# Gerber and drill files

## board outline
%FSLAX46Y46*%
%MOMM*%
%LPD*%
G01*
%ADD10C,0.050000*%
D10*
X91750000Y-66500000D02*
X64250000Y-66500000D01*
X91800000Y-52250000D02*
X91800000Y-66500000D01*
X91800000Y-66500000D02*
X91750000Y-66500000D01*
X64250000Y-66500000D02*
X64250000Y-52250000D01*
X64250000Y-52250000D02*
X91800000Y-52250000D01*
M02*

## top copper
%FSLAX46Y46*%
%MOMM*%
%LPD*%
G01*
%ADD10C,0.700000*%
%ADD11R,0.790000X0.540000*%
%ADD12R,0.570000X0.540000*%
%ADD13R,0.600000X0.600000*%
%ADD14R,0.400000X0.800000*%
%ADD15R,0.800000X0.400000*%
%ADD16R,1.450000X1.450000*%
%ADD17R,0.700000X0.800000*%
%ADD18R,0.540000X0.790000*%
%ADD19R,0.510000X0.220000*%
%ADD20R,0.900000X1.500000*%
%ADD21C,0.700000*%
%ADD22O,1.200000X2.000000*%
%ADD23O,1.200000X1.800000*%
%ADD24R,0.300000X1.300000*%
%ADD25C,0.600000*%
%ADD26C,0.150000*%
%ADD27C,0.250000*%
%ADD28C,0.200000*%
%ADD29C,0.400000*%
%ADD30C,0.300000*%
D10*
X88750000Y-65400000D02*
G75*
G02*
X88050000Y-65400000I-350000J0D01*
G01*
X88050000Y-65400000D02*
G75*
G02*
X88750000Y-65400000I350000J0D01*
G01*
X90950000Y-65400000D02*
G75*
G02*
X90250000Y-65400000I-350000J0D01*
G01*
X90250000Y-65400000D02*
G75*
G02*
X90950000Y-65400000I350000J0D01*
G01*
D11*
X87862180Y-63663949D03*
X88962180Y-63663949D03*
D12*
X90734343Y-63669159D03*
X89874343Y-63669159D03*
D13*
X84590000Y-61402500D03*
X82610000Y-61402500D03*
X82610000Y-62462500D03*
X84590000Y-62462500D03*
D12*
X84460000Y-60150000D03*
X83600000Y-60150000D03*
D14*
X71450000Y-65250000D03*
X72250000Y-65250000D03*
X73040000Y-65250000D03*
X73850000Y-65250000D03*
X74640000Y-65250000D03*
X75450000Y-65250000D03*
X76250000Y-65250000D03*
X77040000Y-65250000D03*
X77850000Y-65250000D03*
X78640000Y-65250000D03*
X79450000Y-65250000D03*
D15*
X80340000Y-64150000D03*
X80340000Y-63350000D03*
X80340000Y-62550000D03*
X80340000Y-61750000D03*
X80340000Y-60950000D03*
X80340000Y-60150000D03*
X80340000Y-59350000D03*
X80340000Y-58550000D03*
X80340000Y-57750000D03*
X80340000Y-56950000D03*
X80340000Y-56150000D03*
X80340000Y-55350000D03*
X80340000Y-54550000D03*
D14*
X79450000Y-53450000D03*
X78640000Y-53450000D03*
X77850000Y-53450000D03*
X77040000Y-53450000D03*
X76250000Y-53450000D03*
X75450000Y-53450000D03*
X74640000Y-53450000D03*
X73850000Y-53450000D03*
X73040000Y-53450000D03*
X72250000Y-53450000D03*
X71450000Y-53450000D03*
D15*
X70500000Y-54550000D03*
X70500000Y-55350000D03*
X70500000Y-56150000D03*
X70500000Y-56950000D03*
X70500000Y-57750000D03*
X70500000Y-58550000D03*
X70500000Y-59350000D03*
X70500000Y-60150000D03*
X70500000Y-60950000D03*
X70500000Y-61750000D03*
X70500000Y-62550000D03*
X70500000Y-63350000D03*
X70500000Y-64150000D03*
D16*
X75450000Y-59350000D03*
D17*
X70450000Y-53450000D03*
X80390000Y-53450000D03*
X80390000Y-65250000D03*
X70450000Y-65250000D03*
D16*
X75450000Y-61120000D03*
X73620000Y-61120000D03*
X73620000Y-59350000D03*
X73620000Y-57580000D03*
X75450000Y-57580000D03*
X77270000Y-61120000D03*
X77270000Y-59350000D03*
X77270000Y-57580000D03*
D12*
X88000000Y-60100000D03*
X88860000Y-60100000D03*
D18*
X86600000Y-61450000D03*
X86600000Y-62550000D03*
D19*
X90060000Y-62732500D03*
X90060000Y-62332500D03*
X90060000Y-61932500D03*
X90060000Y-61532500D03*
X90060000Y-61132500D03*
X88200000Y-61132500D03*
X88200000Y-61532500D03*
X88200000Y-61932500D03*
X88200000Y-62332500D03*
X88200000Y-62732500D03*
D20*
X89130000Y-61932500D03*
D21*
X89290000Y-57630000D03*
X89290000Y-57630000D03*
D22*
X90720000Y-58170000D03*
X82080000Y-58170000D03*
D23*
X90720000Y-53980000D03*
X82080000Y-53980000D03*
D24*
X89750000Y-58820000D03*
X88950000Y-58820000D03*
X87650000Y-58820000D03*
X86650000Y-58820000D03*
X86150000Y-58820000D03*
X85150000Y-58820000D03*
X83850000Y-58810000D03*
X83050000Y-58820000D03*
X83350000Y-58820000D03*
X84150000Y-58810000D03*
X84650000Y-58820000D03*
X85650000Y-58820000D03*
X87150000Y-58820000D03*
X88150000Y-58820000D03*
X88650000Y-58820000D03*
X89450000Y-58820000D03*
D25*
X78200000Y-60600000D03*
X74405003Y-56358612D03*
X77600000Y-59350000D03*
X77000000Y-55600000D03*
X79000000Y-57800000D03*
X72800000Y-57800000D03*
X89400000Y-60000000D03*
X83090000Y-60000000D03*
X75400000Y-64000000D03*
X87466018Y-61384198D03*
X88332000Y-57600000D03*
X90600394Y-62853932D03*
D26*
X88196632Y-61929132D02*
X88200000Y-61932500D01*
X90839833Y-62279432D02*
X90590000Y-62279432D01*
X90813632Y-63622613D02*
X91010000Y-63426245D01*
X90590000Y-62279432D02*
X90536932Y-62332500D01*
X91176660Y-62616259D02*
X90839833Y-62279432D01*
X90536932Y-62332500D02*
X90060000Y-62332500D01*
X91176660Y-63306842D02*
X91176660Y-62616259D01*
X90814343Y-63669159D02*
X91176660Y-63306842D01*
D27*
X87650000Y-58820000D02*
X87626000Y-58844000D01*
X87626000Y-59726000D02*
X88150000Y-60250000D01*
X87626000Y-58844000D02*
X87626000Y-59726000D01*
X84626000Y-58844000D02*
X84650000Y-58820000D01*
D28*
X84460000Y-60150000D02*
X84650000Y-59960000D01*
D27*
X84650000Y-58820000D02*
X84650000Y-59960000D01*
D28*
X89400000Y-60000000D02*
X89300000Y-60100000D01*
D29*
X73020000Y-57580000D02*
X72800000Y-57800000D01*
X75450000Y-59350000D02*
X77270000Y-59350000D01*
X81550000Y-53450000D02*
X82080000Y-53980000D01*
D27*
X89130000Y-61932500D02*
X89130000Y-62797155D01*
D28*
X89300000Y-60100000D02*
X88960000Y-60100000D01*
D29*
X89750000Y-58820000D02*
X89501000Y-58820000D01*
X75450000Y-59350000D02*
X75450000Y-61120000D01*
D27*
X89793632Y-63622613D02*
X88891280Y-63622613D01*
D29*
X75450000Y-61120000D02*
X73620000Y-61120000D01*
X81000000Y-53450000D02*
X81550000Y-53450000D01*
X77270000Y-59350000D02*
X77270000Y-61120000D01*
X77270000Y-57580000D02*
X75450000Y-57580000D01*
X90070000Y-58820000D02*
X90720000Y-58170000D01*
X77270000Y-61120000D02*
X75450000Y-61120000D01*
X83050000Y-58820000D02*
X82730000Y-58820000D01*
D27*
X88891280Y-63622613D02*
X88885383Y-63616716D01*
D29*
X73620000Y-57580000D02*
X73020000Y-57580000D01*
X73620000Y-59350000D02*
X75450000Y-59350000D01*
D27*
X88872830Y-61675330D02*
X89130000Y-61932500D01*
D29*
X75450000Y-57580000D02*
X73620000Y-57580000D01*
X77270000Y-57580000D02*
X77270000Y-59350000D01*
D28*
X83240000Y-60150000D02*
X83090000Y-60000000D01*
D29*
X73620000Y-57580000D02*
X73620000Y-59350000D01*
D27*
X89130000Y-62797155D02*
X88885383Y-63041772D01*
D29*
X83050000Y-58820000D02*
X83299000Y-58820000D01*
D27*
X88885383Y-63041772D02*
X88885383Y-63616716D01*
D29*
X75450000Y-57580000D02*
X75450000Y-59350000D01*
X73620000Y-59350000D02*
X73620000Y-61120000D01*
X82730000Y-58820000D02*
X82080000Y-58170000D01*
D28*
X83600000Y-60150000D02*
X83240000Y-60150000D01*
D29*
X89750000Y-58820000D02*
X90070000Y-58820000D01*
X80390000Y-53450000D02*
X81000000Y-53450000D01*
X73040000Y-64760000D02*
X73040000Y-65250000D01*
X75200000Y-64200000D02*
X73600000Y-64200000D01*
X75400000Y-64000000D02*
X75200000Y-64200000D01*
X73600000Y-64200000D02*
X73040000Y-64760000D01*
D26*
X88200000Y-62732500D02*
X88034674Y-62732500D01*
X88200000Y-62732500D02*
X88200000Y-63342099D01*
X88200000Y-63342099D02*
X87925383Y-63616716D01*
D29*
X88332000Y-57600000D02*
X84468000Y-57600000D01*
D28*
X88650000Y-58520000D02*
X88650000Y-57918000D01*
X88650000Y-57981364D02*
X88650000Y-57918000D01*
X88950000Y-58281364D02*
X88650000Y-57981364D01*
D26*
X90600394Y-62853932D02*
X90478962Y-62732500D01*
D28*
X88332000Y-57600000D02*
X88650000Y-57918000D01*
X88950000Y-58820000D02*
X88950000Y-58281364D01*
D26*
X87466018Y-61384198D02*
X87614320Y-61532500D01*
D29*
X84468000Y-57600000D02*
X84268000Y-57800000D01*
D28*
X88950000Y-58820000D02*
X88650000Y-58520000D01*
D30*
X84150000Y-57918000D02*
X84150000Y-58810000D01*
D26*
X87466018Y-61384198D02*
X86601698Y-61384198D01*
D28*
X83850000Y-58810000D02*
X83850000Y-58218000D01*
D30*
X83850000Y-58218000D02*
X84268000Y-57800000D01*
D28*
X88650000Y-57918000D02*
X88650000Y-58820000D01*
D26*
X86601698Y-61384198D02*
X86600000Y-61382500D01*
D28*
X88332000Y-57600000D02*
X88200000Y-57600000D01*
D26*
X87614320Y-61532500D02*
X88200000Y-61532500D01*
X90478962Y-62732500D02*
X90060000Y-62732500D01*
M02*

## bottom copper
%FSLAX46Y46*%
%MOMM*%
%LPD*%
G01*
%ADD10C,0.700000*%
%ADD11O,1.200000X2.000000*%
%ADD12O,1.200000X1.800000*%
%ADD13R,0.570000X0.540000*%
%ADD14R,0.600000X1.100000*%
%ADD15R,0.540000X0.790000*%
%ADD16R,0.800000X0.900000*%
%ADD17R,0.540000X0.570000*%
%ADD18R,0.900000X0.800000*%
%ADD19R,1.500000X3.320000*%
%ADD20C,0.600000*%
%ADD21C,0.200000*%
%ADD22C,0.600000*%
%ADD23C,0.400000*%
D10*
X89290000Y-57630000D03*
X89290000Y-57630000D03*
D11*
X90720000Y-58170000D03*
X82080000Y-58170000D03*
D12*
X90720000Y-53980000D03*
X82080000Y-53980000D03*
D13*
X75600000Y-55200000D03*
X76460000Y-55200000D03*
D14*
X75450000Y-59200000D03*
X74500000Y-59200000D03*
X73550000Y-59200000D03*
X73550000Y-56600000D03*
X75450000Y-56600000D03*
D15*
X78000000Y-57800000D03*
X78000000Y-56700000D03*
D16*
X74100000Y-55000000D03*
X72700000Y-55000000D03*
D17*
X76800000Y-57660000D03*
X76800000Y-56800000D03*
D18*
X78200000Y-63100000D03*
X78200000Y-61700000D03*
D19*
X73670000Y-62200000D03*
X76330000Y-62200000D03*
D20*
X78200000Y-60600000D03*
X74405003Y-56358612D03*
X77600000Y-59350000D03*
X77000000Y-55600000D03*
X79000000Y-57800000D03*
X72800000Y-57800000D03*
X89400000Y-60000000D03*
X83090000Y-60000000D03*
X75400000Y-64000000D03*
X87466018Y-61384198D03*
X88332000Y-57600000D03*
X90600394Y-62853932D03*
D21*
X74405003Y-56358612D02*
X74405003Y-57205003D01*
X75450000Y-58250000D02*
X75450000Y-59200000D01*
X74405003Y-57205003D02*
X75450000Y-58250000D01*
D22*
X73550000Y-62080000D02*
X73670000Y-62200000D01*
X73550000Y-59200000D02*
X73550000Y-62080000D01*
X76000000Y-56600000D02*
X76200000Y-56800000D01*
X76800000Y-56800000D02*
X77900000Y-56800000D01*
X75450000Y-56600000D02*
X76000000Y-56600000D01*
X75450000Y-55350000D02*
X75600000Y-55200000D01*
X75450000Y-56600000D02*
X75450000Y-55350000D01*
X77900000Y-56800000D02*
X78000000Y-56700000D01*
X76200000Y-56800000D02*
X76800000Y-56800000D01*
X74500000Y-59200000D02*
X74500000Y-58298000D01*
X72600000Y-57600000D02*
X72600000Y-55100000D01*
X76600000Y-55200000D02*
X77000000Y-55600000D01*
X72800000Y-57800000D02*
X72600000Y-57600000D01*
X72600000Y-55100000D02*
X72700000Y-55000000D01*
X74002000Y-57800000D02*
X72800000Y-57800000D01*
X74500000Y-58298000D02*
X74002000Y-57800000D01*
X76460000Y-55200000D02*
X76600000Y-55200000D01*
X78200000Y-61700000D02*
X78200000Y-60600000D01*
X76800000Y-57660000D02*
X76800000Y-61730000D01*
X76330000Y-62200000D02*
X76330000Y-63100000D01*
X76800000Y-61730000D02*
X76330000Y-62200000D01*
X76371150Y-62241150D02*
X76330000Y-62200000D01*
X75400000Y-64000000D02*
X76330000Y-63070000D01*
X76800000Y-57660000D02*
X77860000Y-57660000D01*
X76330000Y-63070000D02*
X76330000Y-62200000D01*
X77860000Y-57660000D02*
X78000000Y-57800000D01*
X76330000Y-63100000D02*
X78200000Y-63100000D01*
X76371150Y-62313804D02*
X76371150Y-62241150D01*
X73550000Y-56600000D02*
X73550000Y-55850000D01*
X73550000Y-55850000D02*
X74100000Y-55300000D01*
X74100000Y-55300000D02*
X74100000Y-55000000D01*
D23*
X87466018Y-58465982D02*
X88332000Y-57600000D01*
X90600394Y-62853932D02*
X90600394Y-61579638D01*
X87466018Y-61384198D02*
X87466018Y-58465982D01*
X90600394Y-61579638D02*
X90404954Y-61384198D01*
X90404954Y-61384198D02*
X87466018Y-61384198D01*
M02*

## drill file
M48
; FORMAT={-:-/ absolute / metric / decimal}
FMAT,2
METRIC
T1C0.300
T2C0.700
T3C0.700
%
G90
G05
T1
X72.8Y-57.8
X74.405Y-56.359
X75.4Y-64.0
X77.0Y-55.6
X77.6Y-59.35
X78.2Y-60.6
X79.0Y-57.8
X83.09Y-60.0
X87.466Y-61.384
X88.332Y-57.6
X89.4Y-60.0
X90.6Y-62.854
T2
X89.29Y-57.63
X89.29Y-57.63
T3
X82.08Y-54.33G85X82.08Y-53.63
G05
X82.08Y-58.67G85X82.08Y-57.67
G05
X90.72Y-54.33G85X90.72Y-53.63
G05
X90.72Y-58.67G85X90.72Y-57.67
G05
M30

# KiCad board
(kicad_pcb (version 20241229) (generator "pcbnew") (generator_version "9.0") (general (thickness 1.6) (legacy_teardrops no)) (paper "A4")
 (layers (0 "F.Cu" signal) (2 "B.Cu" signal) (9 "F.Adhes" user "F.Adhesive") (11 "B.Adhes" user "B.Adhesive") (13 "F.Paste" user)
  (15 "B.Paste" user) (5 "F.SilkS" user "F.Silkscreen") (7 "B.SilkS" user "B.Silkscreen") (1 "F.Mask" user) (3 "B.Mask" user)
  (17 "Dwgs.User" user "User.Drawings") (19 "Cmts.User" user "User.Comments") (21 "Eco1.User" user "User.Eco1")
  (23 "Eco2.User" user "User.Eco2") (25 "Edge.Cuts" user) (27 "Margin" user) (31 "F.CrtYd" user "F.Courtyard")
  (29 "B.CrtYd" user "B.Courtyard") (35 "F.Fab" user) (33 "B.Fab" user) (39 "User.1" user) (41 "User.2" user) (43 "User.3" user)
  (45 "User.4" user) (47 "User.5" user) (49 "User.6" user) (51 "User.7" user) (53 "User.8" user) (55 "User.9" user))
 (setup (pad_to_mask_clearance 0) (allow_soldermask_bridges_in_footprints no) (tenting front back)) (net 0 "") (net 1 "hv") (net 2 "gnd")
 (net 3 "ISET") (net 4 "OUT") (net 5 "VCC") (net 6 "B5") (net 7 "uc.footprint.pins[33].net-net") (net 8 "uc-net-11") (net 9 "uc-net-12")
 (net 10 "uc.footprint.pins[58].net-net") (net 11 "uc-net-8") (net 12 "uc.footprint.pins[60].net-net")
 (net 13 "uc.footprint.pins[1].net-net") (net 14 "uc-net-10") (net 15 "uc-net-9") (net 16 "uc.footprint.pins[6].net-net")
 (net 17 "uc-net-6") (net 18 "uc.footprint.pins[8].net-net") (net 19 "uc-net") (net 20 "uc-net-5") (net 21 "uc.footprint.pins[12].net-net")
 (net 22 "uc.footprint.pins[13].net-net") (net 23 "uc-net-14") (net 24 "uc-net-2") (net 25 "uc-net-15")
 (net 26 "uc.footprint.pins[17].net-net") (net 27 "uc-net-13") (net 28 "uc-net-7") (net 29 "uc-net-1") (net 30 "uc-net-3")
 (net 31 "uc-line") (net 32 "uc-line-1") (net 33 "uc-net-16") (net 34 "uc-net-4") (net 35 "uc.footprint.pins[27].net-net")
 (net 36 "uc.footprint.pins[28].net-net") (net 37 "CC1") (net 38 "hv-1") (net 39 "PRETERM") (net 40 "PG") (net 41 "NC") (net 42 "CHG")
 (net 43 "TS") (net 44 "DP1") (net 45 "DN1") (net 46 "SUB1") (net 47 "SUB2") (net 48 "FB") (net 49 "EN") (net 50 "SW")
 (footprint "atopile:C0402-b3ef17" (layer "F.Cu") (at 88.41218 63.663949)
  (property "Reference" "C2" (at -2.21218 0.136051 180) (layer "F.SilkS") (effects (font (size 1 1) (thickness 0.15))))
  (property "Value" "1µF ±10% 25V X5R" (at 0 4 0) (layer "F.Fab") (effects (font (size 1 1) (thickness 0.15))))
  (pad "1" smd rect (at -0.55 0) (size 0.79 0.54) (layers "F.Cu" "F.Mask" "F.Paste") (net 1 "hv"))
  (pad "2" smd rect (at 0.55 0) (size 0.79 0.54) (layers "F.Cu" "F.Mask" "F.Paste") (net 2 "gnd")))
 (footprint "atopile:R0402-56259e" (layer "F.Cu") (at 90.304343 63.669159 180)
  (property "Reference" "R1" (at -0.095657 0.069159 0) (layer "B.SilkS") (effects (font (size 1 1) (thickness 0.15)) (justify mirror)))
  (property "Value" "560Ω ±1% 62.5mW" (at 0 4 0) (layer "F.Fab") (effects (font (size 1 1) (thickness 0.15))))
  (pad "1" smd rect (at -0.43 0 180) (size 0.57 0.54) (layers "F.Cu" "F.Mask" "F.Paste") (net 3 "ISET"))
  (pad "2" smd rect (at 0.43 0 180) (size 0.57 0.54) (layers "F.Cu" "F.Mask" "F.Paste") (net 2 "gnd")))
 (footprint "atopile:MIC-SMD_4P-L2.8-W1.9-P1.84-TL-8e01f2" (layer "F.Cu") (at 83.6 61.9325 -90)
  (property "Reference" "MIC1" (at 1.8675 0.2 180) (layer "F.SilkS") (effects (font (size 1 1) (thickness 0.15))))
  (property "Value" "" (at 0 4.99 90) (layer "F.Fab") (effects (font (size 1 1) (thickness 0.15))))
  (pad "1" smd rect (at -0.53 -0.99 270) (size 0.6 0.6) (layers "F.Cu" "F.Mask" "F.Paste") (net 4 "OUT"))
  (pad "2" smd rect (at -0.53 0.99 270) (size 0.6 0.6) (layers "F.Cu" "F.Mask" "F.Paste") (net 2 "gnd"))
  (pad "3" smd rect (at 0.53 0.99 270) (size 0.6 0.6) (layers "F.Cu" "F.Mask" "F.Paste") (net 2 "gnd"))
  (pad "4" smd rect (at 0.53 -0.99 270) (size 0.6 0.6) (layers "F.Cu" "F.Mask" "F.Paste") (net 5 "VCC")))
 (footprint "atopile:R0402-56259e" (layer "F.Cu") (at 84.03 60.15 180)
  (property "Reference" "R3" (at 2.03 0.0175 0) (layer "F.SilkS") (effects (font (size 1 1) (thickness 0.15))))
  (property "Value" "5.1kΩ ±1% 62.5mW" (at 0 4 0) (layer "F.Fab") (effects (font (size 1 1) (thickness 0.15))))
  (pad "1" smd rect (at -0.43 0 180) (size 0.57 0.54) (layers "F.Cu" "F.Mask" "F.Paste") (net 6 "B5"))
  (pad "2" smd rect (at 0.43 0 180) (size 0.57 0.54) (layers "F.Cu" "F.Mask" "F.Paste") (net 2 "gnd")))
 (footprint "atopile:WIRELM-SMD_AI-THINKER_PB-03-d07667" (layer "F.Cu") (at 75.42 59.35 90)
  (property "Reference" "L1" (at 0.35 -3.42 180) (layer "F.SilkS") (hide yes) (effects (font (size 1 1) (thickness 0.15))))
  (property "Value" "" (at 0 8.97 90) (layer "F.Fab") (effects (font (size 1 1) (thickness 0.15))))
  (pad "1" smd rect (at -5.9 -3.97 180) (size 0.4 0.8) (layers "F.Cu" "F.Mask" "F.Paste") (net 2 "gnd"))
  (pad "2" smd rect (at -5.9 -3.17 180) (size 0.4 0.8) (layers "F.Cu" "F.Mask" "F.Paste") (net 2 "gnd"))
  (pad "3" smd rect (at -5.9 -2.38 180) (size 0.4 0.8) (layers "F.Cu" "F.Mask" "F.Paste") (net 5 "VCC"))
  (pad "4" smd rect (at -5.9 -1.57 180) (size 0.4 0.8) (layers "F.Cu" "F.Mask" "F.Paste") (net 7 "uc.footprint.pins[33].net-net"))
  (pad "5" smd rect (at -5.9 -0.78 180) (size 0.4 0.8) (layers "F.Cu" "F.Mask" "F.Paste") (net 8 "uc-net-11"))
  (pad "6" smd rect (at -5.9 0.03 180) (size 0.4 0.8) (layers "F.Cu" "F.Mask" "F.Paste") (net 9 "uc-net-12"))
  (pad "7" smd rect (at -5.9 0.83 180) (size 0.4 0.8) (layers "F.Cu" "F.Mask" "F.Paste") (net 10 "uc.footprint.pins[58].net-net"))
  (pad "8" smd rect (at -5.9 1.62 180) (size 0.4 0.8) (layers "F.Cu" "F.Mask" "F.Paste") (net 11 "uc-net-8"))
  (pad "9" smd rect (at -5.9 2.43 180) (size 0.4 0.8) (layers "F.Cu" "F.Mask" "F.Paste") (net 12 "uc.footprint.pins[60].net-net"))
  (pad "10" smd rect (at -5.9 3.22 180) (size 0.4 0.8) (layers "F.Cu" "F.Mask" "F.Paste") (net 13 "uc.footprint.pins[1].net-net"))
  (pad "11" smd rect (at -5.9 4.03 180) (size 0.4 0.8) (layers "F.Cu" "F.Mask" "F.Paste") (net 2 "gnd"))
  (pad "12" smd rect (at -4.8 4.92 270) (size 0.4 0.8) (layers "F.Cu" "F.Mask" "F.Paste") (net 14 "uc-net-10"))
  (pad "13" smd rect (at -4 4.92 270) (size 0.4 0.8) (layers "F.Cu" "F.Mask" "F.Paste") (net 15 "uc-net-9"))
  (pad "14" smd rect (at -3.2 4.92 270) (size 0.4 0.8) (layers "F.Cu" "F.Mask" "F.Paste") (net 2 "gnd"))
  (pad "15" smd rect (at -2.4 4.92 270) (size 0.4 0.8) (layers "F.Cu" "F.Mask" "F.Paste") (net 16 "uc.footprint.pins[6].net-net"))
  (pad "16" smd rect (at -1.6 4.92 270) (size 0.4 0.8) (layers "F.Cu" "F.Mask" "F.Paste") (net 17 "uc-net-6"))
  (pad "17" smd rect (at -0.8 4.92 270) (size 0.4 0.8) (layers "F.Cu" "F.Mask" "F.Paste") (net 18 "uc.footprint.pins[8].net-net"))
  (pad "18" smd rect (at 0 4.92 270) (size 0.4 0.8) (layers "F.Cu" "F.Mask" "F.Paste") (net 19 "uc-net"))
  (pad "19" smd rect (at 0.8 4.92 270) (size 0.4 0.8) (layers "F.Cu" "F.Mask" "F.Paste") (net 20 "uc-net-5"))
  (pad "20" smd rect (at 1.6 4.92 270) (size 0.4 0.8) (layers "F.Cu" "F.Mask" "F.Paste") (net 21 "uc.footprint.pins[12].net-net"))
  (pad "21" smd rect (at 2.4 4.92 270) (size 0.4 0.8) (layers "F.Cu" "F.Mask" "F.Paste") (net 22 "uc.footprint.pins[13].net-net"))
  (pad "22" smd rect (at 3.2 4.92 270) (size 0.4 0.8) (layers "F.Cu" "F.Mask" "F.Paste") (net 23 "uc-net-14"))
  (pad "23" smd rect (at 4 4.92 270) (size 0.4 0.8) (layers "F.Cu" "F.Mask" "F.Paste") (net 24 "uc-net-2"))
  (pad "24" smd rect (at 4.8 4.92 270) (size 0.4 0.8) (layers "F.Cu" "F.Mask" "F.Paste") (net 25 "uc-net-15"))
  (pad "25" smd rect (at 5.9 4.03) (size 0.4 0.8) (layers "F.Cu" "F.Mask" "F.Paste") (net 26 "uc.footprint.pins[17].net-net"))
  (pad "26" smd rect (at 5.9 3.22) (size 0.4 0.8) (layers "F.Cu" "F.Mask" "F.Paste") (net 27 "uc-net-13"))
  (pad "27" smd rect (at 5.9 2.43) (size 0.4 0.8) (layers "F.Cu" "F.Mask" "F.Paste") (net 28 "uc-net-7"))
  (pad "28" smd rect (at 5.9 1.62) (size 0.4 0.8) (layers "F.Cu" "F.Mask" "F.Paste") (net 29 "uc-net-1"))
  (pad "29" smd rect (at 5.9 0.83) (size 0.4 0.8) (layers "F.Cu" "F.Mask" "F.Paste") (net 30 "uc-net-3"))
  (pad "30" smd rect (at 5.9 0.03) (size 0.4 0.8) (layers "F.Cu" "F.Mask" "F.Paste") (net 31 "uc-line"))
  (pad "31" smd rect (at 5.9 -0.78) (size 0.4 0.8) (layers "F.Cu" "F.Mask" "F.Paste") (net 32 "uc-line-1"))
  (pad "32" smd rect (at 5.9 -1.57) (size 0.4 0.8) (layers "F.Cu" "F.Mask" "F.Paste") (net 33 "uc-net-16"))
  (pad "33" smd rect (at 5.9 -2.38) (size 0.4 0.8) (layers "F.Cu" "F.Mask" "F.Paste") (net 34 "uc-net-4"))
  (pad "34" smd rect (at 5.9 -3.17) (size 0.4 0.8) (layers "F.Cu" "F.Mask" "F.Paste") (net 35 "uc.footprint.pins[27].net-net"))
  (pad "35" smd rect (at 5.9 -3.97) (size 0.4 0.8) (layers "F.Cu" "F.Mask" "F.Paste") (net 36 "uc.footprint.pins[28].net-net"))
  (pad "36" smd rect (at 4.8 -4.92 90) (size 0.4 0.8) (layers "F.Cu" "F.Mask" "F.Paste") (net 2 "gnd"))
  (pad "37" smd rect (at 4 -4.92 90) (size 0.4 0.8) (layers "F.Cu" "F.Mask" "F.Paste") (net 2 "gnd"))
  (pad "38" smd rect (at 3.2 -4.92 90) (size 0.4 0.8) (layers "F.Cu" "F.Mask" "F.Paste") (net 2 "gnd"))
  (pad "39" smd rect (at 2.4 -4.92 90) (size 0.4 0.8) (layers "F.Cu" "F.Mask" "F.Paste") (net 2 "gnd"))
  (pad "40" smd rect (at 1.6 -4.92 90) (size 0.4 0.8) (layers "F.Cu" "F.Mask" "F.Paste") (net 2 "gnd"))
  (pad "41" smd rect (at 0.8 -4.92 90) (size 0.4 0.8) (layers "F.Cu" "F.Mask" "F.Paste") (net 2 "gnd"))
  (pad "42" smd rect (at 0 -4.92 90) (size 0.4 0.8) (layers "F.Cu" "F.Mask" "F.Paste") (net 2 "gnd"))
  (pad "43" smd rect (at -0.8 -4.92 90) (size 0.4 0.8) (layers "F.Cu" "F.Mask" "F.Paste") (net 2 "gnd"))
  (pad "44" smd rect (at -1.6 -4.92 90) (size 0.4 0.8) (layers "F.Cu" "F.Mask" "F.Paste") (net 2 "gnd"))
  (pad "45" smd rect (at -2.4 -4.92 90) (size 0.4 0.8) (layers "F.Cu" "F.Mask" "F.Paste") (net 2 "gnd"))
  (pad "46" smd rect (at -3.2 -4.92 90) (size 0.4 0.8) (layers "F.Cu" "F.Mask" "F.Paste") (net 2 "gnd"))
  (pad "47" smd rect (at -4 -4.92 90) (size 0.4 0.8) (layers "F.Cu" "F.Mask" "F.Paste") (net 2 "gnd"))
  (pad "48" smd rect (at -4.8 -4.92 90) (size 0.4 0.8) (layers "F.Cu" "F.Mask" "F.Paste") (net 2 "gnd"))
  (pad "49" smd rect (at 0 0.03 90) (size 1.45 1.45) (layers "F.Cu" "F.Mask" "F.Paste") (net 2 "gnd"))
  (pad "50" smd rect (at 5.9 -4.97 180) (size 0.7 0.8) (layers "F.Cu" "F.Mask" "F.Paste") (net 2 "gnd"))
  (pad "51" smd rect (at 5.9 4.97 180) (size 0.7 0.8) (layers "F.Cu" "F.Mask" "F.Paste") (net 2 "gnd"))
  (pad "52" smd rect (at -5.9 4.97 180) (size 0.7 0.8) (layers "F.Cu" "F.Mask" "F.Paste") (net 2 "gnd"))
  (pad "53" smd rect (at -5.9 -4.97 180) (size 0.7 0.8) (layers "F.Cu" "F.Mask" "F.Paste") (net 2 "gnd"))
  (pad "54" smd rect (at -1.77 0.03 90) (size 1.45 1.45) (layers "F.Cu" "F.Mask" "F.Paste") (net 2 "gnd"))
  (pad "55" smd rect (at -1.77 -1.8 90) (size 1.45 1.45) (layers "F.Cu" "F.Mask" "F.Paste") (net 2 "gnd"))
  (pad "56" smd rect (at 0 -1.8 90) (size 1.45 1.45) (layers "F.Cu" "F.Mask" "F.Paste") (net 2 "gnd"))
  (pad "57" smd rect (at 1.77 -1.8 90) (size 1.45 1.45) (layers "F.Cu" "F.Mask" "F.Paste") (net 2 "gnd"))
  (pad "58" smd rect (at 1.77 0.03 90) (size 1.45 1.45) (layers "F.Cu" "F.Mask" "F.Paste") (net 2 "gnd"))
  (pad "59" smd rect (at -1.77 1.85 90) (size 1.45 1.45) (layers "F.Cu" "F.Mask" "F.Paste") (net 2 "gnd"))
  (pad "60" smd rect (at 0 1.85 90) (size 1.45 1.45) (layers "F.Cu" "F.Mask" "F.Paste") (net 2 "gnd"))
  (pad "61" smd rect (at 1.77 1.85 90) (size 1.45 1.45) (layers "F.Cu" "F.Mask" "F.Paste") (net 2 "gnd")))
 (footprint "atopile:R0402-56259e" (layer "F.Cu") (at 88.43 60.1)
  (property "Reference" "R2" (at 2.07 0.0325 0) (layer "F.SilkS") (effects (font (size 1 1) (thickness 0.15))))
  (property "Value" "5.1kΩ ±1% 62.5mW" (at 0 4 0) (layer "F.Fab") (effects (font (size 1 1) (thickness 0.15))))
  (pad "1" smd rect (at -0.43 0) (size 0.57 0.54) (layers "F.Cu" "F.Mask" "F.Paste") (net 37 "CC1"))
  (pad "2" smd rect (at 0.43 0) (size 0.57 0.54) (layers "F.Cu" "F.Mask" "F.Paste") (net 2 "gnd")))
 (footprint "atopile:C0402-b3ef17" (layer "F.Cu") (at 86.6 62 -90)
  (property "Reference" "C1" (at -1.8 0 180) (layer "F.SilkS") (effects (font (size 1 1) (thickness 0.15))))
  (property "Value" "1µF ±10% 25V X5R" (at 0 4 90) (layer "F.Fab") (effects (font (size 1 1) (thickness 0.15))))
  (pad "1" smd rect (at -0.55 0 270) (size 0.79 0.54) (layers "F.Cu" "F.Mask" "F.Paste") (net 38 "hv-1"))
  (pad "2" smd rect (at 0.55 0 270) (size 0.79 0.54) (layers "F.Cu" "F.Mask" "F.Paste") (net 2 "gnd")))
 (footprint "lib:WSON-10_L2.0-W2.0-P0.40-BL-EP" (layer "F.Cu") (at 89.13 61.9325 90)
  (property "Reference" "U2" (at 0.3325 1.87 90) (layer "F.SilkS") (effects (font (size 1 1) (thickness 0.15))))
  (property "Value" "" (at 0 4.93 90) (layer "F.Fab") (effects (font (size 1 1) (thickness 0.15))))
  (pad "1" smd rect (at -0.8 0.93 90) (size 0.22 0.51) (layers "F.Cu" "F.Mask" "F.Paste") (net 38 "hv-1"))
  (pad "2" smd rect (at -0.4 0.93 90) (size 0.22 0.51) (layers "F.Cu" "F.Mask" "F.Paste") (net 3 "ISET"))
  (pad "3" smd rect (at 0 0.93 90) (size 0.22 0.51) (layers "F.Cu" "F.Mask" "F.Paste") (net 2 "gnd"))
  (pad "4" smd rect (at 0.4 0.93 90) (size 0.22 0.51) (layers "F.Cu" "F.Mask" "F.Paste") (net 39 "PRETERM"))
  (pad "5" smd rect (at 0.8 0.93 90) (size 0.22 0.51) (layers "F.Cu" "F.Mask" "F.Paste") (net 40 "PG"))
  (pad "6" smd rect (at 0.8 -0.93 90) (size 0.22 0.51) (layers "F.Cu" "F.Mask" "F.Paste") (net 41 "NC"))
  (pad "7" smd rect (at 0.4 -0.93 90) (size 0.22 0.51) (layers "F.Cu" "F.Mask" "F.Paste") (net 38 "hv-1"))
  (pad "8" smd rect (at 0 -0.93 90) (size 0.22 0.51) (layers "F.Cu" "F.Mask" "F.Paste") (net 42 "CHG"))
  (pad "9" smd rect (at -0.4 -0.93 90) (size 0.22 0.51) (layers "F.Cu" "F.Mask" "F.Paste") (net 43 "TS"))
  (pad "10" smd rect (at -0.8 -0.93 90) (size 0.22 0.51) (layers "F.Cu" "F.Mask" "F.Paste") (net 1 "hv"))
  (pad "11" smd rect (at 0 0 90) (size 1.5 0.9) (layers "F.Cu" "F.Mask" "F.Paste") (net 2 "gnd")))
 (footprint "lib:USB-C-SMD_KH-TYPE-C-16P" (layer "F.Cu") (at 86.4 56.4 180)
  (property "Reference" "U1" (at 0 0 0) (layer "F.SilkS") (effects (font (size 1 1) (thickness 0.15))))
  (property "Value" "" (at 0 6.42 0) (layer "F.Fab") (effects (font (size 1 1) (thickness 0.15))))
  (pad "" thru_hole circle (at -2.89 -1.23 180) (size 0.7 0.7) (drill 0.7) (layers "*.Cu" "*.Mask") (remove_unused_layers no))
  (pad "" thru_hole circle (at -2.89 -1.23 180) (size 0.7 0.7) (drill 0.7) (layers "*.Cu" "*.Mask") (remove_unused_layers no))
  (pad "1" thru_hole oval (at -4.32 -1.77 180) (size 1.2 2) (drill oval 0.700024 1.699997) (layers "*.Cu" "*.Mask")
   (remove_unused_layers no) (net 2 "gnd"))
  (pad "2" thru_hole oval (at 4.32 -1.77 180) (size 1.2 2) (drill oval 0.700024 1.699997) (layers "*.Cu" "*.Mask") (remove_unused_layers no)
   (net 2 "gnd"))
  (pad "3" thru_hole oval (at -4.32 2.42 180) (size 1.2 1.8) (drill oval 0.700024 1.399997) (layers "*.Cu" "*.Mask")
   (remove_unused_layers no) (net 2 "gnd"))
  (pad "4" thru_hole oval (at 4.32 2.42 180) (size 1.2 1.8) (drill oval 0.700024 1.399997) (layers "*.Cu" "*.Mask")
   (remove_unused_layers no) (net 2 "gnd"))
  (pad "A1" smd rect (at -3.35 -2.42 180) (size 0.3 1.3) (layers "F.Cu" "F.Mask" "F.Paste") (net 2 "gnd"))
  (pad "A4" smd rect (at -2.55 -2.42 180) (size 0.3 1.3) (layers "F.Cu" "F.Mask" "F.Paste") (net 38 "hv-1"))
  (pad "A5" smd rect (at -1.25 -2.42 180) (size 0.3 1.3) (layers "F.Cu" "F.Mask" "F.Paste") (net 37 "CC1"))
  (pad "A6" smd rect (at -0.25 -2.42 180) (size 0.3 1.3) (layers "F.Cu" "F.Mask" "F.Paste") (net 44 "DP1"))
  (pad "A7" smd rect (at 0.25 -2.42 180) (size 0.3 1.3) (layers "F.Cu" "F.Mask" "F.Paste") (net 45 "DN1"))
  (pad "A8" smd rect (at 1.25 -2.42 180) (size 0.3 1.3) (layers "F.Cu" "F.Mask" "F.Paste") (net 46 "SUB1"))
  (pad "A9" smd rect (at 2.55 -2.41 180) (size 0.3 1.3) (layers "F.Cu" "F.Mask" "F.Paste") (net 38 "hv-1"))
  (pad "A12" smd rect (at 3.35 -2.42 180) (size 0.3 1.3) (layers "F.Cu" "F.Mask" "F.Paste") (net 2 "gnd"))
  (pad "B1" smd rect (at 3.05 -2.42 180) (size 0.3 1.3) (layers "F.Cu" "F.Mask" "F.Paste") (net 2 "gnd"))
  (pad "B4" smd rect (at 2.25 -2.41 180) (size 0.3 1.3) (layers "F.Cu" "F.Mask" "F.Paste") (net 38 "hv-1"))
  (pad "B5" smd rect (at 1.75 -2.42 180) (size 0.3 1.3) (layers "F.Cu" "F.Mask" "F.Paste") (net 6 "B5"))
  (pad "B6" smd rect (at 0.75 -2.42 180) (size 0.3 1.3) (layers "F.Cu" "F.Mask" "F.Paste") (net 44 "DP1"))
  (pad "B7" smd rect (at -0.75 -2.42 180) (size 0.3 1.3) (layers "F.Cu" "F.Mask" "F.Paste") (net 45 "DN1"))
  (pad "B8" smd rect (at -1.75 -2.42 180) (size 0.3 1.3) (layers "F.Cu" "F.Mask" "F.Paste") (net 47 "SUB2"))
  (pad "B9" smd rect (at -2.25 -2.42 180) (size 0.3 1.3) (layers "F.Cu" "F.Mask" "F.Paste") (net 38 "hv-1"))
  (pad "B12" smd rect (at -3.05 -2.42 180) (size 0.3 1.3) (layers "F.Cu" "F.Mask" "F.Paste") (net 2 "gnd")))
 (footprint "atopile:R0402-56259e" (layer "B.Cu") (at 76.03 55.2)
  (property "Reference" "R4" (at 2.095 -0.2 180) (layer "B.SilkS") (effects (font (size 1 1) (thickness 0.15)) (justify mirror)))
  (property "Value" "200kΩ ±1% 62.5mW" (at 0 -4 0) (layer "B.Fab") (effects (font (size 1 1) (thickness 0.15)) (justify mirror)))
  (pad "1" smd rect (at -0.43 0) (size 0.57 0.54) (layers "B.Cu" "B.Mask" "B.Paste") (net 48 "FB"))
  (pad "2" smd rect (at 0.43 0) (size 0.57 0.54) (layers "B.Cu" "B.Mask" "B.Paste") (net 2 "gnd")))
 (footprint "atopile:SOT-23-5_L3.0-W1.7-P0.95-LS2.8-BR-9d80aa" (layer "B.Cu") (at 74.5 57.9 -90)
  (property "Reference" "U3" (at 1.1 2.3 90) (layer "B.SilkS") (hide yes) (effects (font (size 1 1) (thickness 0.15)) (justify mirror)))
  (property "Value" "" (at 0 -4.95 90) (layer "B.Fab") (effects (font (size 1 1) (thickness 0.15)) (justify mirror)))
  (pad "1" smd rect (at 1.3 -0.95 270) (size 1.1 0.6) (layers "B.Cu" "B.Mask" "B.Paste") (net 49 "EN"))
  (pad "2" smd rect (at 1.3 0 270) (size 1.1 0.6) (layers "B.Cu" "B.Mask" "B.Paste") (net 2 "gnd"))
  (pad "3" smd rect (at 1.3 0.95 270) (size 1.1 0.6) (layers "B.Cu" "B.Mask" "B.Paste") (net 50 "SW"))
  (pad "4" smd rect (at -1.3 0.95 270) (size 1.1 0.6) (layers "B.Cu" "B.Mask" "B.Paste") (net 1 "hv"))
  (pad "5" smd rect (at -1.3 -0.95 270) (size 1.1 0.6) (layers "B.Cu" "B.Mask" "B.Paste") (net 48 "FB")))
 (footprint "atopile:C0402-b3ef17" (layer "B.Cu") (at 78 57.25 90)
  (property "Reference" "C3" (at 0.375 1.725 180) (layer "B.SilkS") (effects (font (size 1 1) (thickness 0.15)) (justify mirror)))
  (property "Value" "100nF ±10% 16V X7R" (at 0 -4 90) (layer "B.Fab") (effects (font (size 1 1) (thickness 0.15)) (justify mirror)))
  (pad "1" smd rect (at -0.55 0 90) (size 0.79 0.54) (layers "B.Cu" "B.Mask" "B.Paste") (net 5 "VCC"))
  (pad "2" smd rect (at 0.55 0 90) (size 0.79 0.54) (layers "B.Cu" "B.Mask" "B.Paste") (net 48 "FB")))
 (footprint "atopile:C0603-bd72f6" (layer "B.Cu") (at 73.4 55 180)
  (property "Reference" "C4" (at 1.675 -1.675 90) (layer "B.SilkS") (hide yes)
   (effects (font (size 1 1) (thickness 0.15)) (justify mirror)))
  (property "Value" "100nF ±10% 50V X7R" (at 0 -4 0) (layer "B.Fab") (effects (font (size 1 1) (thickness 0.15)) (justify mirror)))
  (pad "1" smd rect (at -0.7 0 180) (size 0.8 0.9) (layers "B.Cu" "B.Mask" "B.Paste") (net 1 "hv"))
  (pad "2" smd rect (at 0.7 0 180) (size 0.8 0.9) (layers "B.Cu" "B.Mask" "B.Paste") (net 2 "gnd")))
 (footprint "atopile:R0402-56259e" (layer "B.Cu") (at 76.8 57.23 90)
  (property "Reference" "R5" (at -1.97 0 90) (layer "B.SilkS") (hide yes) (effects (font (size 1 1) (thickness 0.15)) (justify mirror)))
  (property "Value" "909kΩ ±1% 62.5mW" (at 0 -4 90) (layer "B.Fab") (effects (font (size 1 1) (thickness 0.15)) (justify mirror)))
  (pad "1" smd rect (at -0.43 0 90) (size 0.57 0.54) (layers "B.Cu" "B.Mask" "B.Paste") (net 5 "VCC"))
  (pad "2" smd rect (at 0.43 0 90) (size 0.57 0.54) (layers "B.Cu" "B.Mask" "B.Paste") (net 48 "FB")))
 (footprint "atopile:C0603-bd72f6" (layer "B.Cu") (at 78.2 62.4 90)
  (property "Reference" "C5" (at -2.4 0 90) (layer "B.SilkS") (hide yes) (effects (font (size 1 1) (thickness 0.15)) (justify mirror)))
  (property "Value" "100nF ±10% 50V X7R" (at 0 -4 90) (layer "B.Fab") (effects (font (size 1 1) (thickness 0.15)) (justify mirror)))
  (pad "1" smd rect (at -0.7 0 90) (size 0.8 0.9) (layers "B.Cu" "B.Mask" "B.Paste") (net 5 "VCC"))
  (pad "2" smd rect (at 0.7 0 90) (size 0.8 0.9) (layers "B.Cu" "B.Mask" "B.Paste") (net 2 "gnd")))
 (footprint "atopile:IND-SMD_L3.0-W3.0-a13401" (layer "B.Cu") (at 75 62.2 180)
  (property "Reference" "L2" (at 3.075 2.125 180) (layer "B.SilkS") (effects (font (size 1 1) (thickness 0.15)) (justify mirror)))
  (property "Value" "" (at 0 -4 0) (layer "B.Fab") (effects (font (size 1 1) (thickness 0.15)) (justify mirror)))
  (pad "1" smd rect (at 1.33 0 180) (size 1.5 3.32) (layers "B.Cu" "B.Mask" "B.Paste") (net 50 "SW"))
  (pad "2" smd rect (at -1.33 0 180) (size 1.5 3.32) (layers "B.Cu" "B.Mask" "B.Paste") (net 5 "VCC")))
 (gr_circle (center 88.4 65.4) (end 88.4 64.8) (stroke (width 0.2) (type solid)) (fill yes) (layer "F.Cu"))
 (gr_circle (center 90.6 65.4) (end 90.6 64.8) (stroke (width 0.2) (type solid)) (fill yes) (layer "F.Cu"))
 (gr_line (start 91.75 66.5) (end 64.25 66.5) (stroke (width 0.05) (type default)) (layer "Edge.Cuts"))
 (gr_line (start 91.8 52.25) (end 91.8 66.5) (stroke (width 0.05) (type default)) (layer "Edge.Cuts"))
 (gr_line (start 91.8 66.5) (end 91.75 66.5) (stroke (width 0.05) (type default)) (layer "Edge.Cuts"))
 (gr_line (start 64.25 66.5) (end 64.25 52.25) (stroke (width 0.05) (type default)) (layer "Edge.Cuts"))
 (gr_line (start 64.25 52.25) (end 91.8 52.25) (stroke (width 0.05) (type default)) (layer "Edge.Cuts"))
 (segment (start 88.196632 61.929132) (end 88.2 61.9325) (width 0.15) (layer "F.Cu") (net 42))
 (via (at 78.2 60.6) (size 0.6) (drill 0.3) (layers "F.Cu" "B.Cu") (free yes) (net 42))
 (segment (start 90.839833 62.279432) (end 90.59 62.279432) (width 0.15) (layer "F.Cu") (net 3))
 (segment (start 90.813632 63.622613) (end 91.01 63.426245) (width 0.15) (layer "F.Cu") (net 3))
 (segment (start 90.59 62.279432) (end 90.536932 62.3325) (width 0.15) (layer "F.Cu") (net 3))
 (segment (start 91.17666 62.616259) (end 90.839833 62.279432) (width 0.15) (layer "F.Cu") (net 3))
 (segment (start 90.536932 62.3325) (end 90.06 62.3325) (width 0.15) (layer "F.Cu") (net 3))
 (segment (start 91.17666 63.306842) (end 91.17666 62.616259) (width 0.15) (layer "F.Cu") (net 3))
 (segment (start 90.814343 63.669159) (end 91.17666 63.306842) (width 0.15) (layer "F.Cu") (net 3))
 (segment (start 87.65 58.82) (end 87.626 58.844) (width 0.25) (layer "F.Cu") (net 37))
 (segment (start 87.626 59.726) (end 88.15 60.25) (width 0.25) (layer "F.Cu") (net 37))
 (segment (start 87.626 58.844) (end 87.626 59.726) (width 0.25) (layer "F.Cu") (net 37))
 (segment (start 84.626 58.844) (end 84.65 58.82) (width 0.25) (layer "F.Cu") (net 6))
 (segment (start 84.46 60.15) (end 84.65 59.96) (width 0.2) (layer "F.Cu") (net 6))
 (segment (start 84.65 58.82) (end 84.65 59.96) (width 0.25) (layer "F.Cu") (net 6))
 (via (at 74.405003 56.358612) (size 0.6) (drill 0.3) (layers "F.Cu" "B.Cu") (free yes) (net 49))
 (segment (start 74.405003 56.358612) (end 74.405003 57.205003) (width 0.2) (layer "B.Cu") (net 49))
 (segment (start 75.45 58.25) (end 75.45 59.2) (width 0.2) (layer "B.Cu") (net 49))
 (segment (start 74.405003 57.205003) (end 75.45 58.25) (width 0.2) (layer "B.Cu") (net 49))
 (segment (start 73.55 62.08) (end 73.67 62.2) (width 0.6) (layer "B.Cu") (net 50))
 (segment (start 73.55 59.2) (end 73.55 62.08) (width 0.6) (layer "B.Cu") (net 50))
 (segment (start 76 56.6) (end 76.2 56.8) (width 0.6) (layer "B.Cu") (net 48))
 (segment (start 76.8 56.8) (end 77.9 56.8) (width 0.6) (layer "B.Cu") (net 48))
 (segment (start 75.45 56.6) (end 76 56.6) (width 0.6) (layer "B.Cu") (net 48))
 (segment (start 75.45 55.35) (end 75.6 55.2) (width 0.6) (layer "B.Cu") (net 48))
 (segment (start 75.45 56.6) (end 75.45 55.35) (width 0.6) (layer "B.Cu") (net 48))
 (segment (start 77.9 56.8) (end 78 56.7) (width 0.6) (layer "B.Cu") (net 48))
 (segment (start 76.2 56.8) (end 76.8 56.8) (width 0.6) (layer "B.Cu") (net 48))
 (segment (start 89.4 60) (end 89.3 60.1) (width 0.2) (layer "F.Cu") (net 2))
 (segment (start 73.02 57.58) (end 72.8 57.8) (width 0.4) (layer "F.Cu") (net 2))
 (segment (start 75.45 59.35) (end 77.27 59.35) (width 0.4) (layer "F.Cu") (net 2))
 (segment (start 81.55 53.45) (end 82.08 53.98) (width 0.4) (layer "F.Cu") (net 2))
 (segment (start 89.13 61.9325) (end 89.13 62.797155) (width 0.25) (layer "F.Cu") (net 2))
 (segment (start 89.3 60.1) (end 88.96 60.1) (width 0.2) (layer "F.Cu") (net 2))
 (segment (start 89.75 58.82) (end 89.501 58.82) (width 0.4) (layer "F.Cu") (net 2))
 (segment (start 75.45 59.35) (end 75.45 61.12) (width 0.4) (layer "F.Cu") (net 2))
 (segment (start 89.793632 63.622613) (end 88.89128 63.622613) (width 0.25) (layer "F.Cu") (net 2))
 (segment (start 75.45 61.12) (end 73.62 61.12) (width 0.4) (layer "F.Cu") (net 2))
 (segment (start 81 53.45) (end 81.55 53.45) (width 0.4) (layer "F.Cu") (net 2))
 (segment (start 77.27 59.35) (end 77.27 61.12) (width 0.4) (layer "F.Cu") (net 2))
 (segment (start 77.27 57.58) (end 75.45 57.58) (width 0.4) (layer "F.Cu") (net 2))
 (segment (start 90.07 58.82) (end 90.72 58.17) (width 0.4) (layer "F.Cu") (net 2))
 (segment (start 77.27 61.12) (end 75.45 61.12) (width 0.4) (layer "F.Cu") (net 2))
 (segment (start 83.05 58.82) (end 82.73 58.82) (width 0.4) (layer "F.Cu") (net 2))
 (segment (start 88.89128 63.622613) (end 88.885383 63.616716) (width 0.25) (layer "F.Cu") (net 2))
 (segment (start 73.62 57.58) (end 73.02 57.58) (width 0.4) (layer "F.Cu") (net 2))
 (segment (start 73.62 59.35) (end 75.45 59.35) (width 0.4) (layer "F.Cu") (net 2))
 (segment (start 88.87283 61.67533) (end 89.13 61.9325) (width 0.25) (layer "F.Cu") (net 2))
 (segment (start 75.45 57.58) (end 73.62 57.58) (width 0.4) (layer "F.Cu") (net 2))
 (segment (start 77.27 57.58) (end 77.27 59.35) (width 0.4) (layer "F.Cu") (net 2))
 (segment (start 83.24 60.15) (end 83.09 60) (width 0.2) (layer "F.Cu") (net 2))
 (segment (start 73.62 57.58) (end 73.62 59.35) (width 0.4) (layer "F.Cu") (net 2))
 (segment (start 89.13 62.797155) (end 88.885383 63.041772) (width 0.25) (layer "F.Cu") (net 2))
 (segment (start 83.05 58.82) (end 83.299 58.82) (width 0.4) (layer "F.Cu") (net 2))
 (segment (start 88.885383 63.041772) (end 88.885383 63.616716) (width 0.25) (layer "F.Cu") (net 2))
 (segment (start 75.45 57.58) (end 75.45 59.35) (width 0.4) (layer "F.Cu") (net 2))
 (segment (start 73.62 59.35) (end 73.62 61.12) (width 0.4) (layer "F.Cu") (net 2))
 (segment (start 82.73 58.82) (end 82.08 58.17) (width 0.4) (layer "F.Cu") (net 2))
 (segment (start 83.6 60.15) (end 83.24 60.15) (width 0.2) (layer "F.Cu") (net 2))
 (segment (start 89.75 58.82) (end 90.07 58.82) (width 0.4) (layer "F.Cu") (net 2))
 (segment (start 80.39 53.45) (end 81 53.45) (width 0.4) (layer "F.Cu") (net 2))
 (via (at 77.6 59.35) (size 0.6) (drill 0.3) (layers "F.Cu" "B.Cu") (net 2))
 (via (at 77 55.6) (size 0.6) (drill 0.3) (layers "F.Cu" "B.Cu") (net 2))
 (via (at 79 57.8) (size 0.6) (drill 0.3) (layers "F.Cu" "B.Cu") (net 2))
 (via (at 72.8 57.8) (size 0.6) (drill 0.3) (layers "F.Cu" "B.Cu") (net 2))
 (via (at 89.4 60) (size 0.6) (drill 0.3) (layers "F.Cu" "B.Cu") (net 2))
 (via (at 83.09 60) (size 0.6) (drill 0.3) (layers "F.Cu" "B.Cu") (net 2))
 (segment (start 74.5 59.2) (end 74.5 58.298) (width 0.6) (layer "B.Cu") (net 2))
 (segment (start 72.6 57.6) (end 72.6 55.1) (width 0.6) (layer "B.Cu") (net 2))
 (segment (start 76.6 55.2) (end 77 55.6) (width 0.6) (layer "B.Cu") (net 2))
 (segment (start 72.8 57.8) (end 72.6 57.6) (width 0.6) (layer "B.Cu") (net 2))
 (segment (start 72.6 55.1) (end 72.7 55) (width 0.6) (layer "B.Cu") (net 2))
 (segment (start 74.002 57.8) (end 72.8 57.8) (width 0.6) (layer "B.Cu") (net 2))
 (segment (start 74.5 58.298) (end 74.002 57.8) (width 0.6) (layer "B.Cu") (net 2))
 (segment (start 76.46 55.2) (end 76.6 55.2) (width 0.6) (layer "B.Cu") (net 2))
 (segment (start 78.2 61.7) (end 78.2 60.6) (width 0.6) (layer "B.Cu") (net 2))
 (segment (start 73.04 64.76) (end 73.04 65.25) (width 0.4) (layer "F.Cu") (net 5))
 (segment (start 75.2 64.2) (end 73.6 64.2) (width 0.4) (layer "F.Cu") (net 5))
 (segment (start 75.4 64) (end 75.2 64.2) (width 0.4) (layer "F.Cu") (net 5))
 (segment (start 73.6 64.2) (end 73.04 64.76) (width 0.4) (layer "F.Cu") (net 5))
 (via (at 75.4 64) (size 0.6) (drill 0.3) (layers "F.Cu" "B.Cu") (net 5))
 (segment (start 76.8 57.66) (end 76.8 61.73) (width 0.6) (layer "B.Cu") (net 5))
 (segment (start 76.33 62.2) (end 76.33 63.1) (width 0.6) (layer "B.Cu") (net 5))
 (segment (start 76.8 61.73) (end 76.33 62.2) (width 0.6) (layer "B.Cu") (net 5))
 (segment (start 76.37115 62.24115) (end 76.33 62.2) (width 0.6) (layer "B.Cu") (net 5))
 (segment (start 75.4 64) (end 76.33 63.07) (width 0.6) (layer "B.Cu") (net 5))
 (segment (start 76.8 57.66) (end 77.86 57.66) (width 0.6) (layer "B.Cu") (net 5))
 (segment (start 76.33 63.07) (end 76.33 62.2) (width 0.6) (layer "B.Cu") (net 5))
 (segment (start 77.86 57.66) (end 78 57.8) (width 0.6) (layer "B.Cu") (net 5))
 (segment (start 76.33 63.1) (end 78.2 63.1) (width 0.6) (layer "B.Cu") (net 5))
 (segment (start 76.37115 62.313804) (end 76.37115 62.24115) (width 0.6) (layer "B.Cu") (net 5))
 (segment (start 88.2 62.7325) (end 88.034674 62.7325) (width 0.15) (layer "F.Cu") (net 1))
 (segment (start 88.2 62.7325) (end 88.2 63.342099) (width 0.15) (layer "F.Cu") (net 1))
 (segment (start 88.2 63.342099) (end 87.925383 63.616716) (width 0.15) (layer "F.Cu") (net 1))
 (segment (start 73.55 56.6) (end 73.55 55.85) (width 0.6) (layer "B.Cu") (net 1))
 (segment (start 73.55 55.85) (end 74.1 55.3) (width 0.6) (layer "B.Cu") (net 1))
 (segment (start 74.1 55.3) (end 74.1 55) (width 0.6) (layer "B.Cu") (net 1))
 (segment (start 88.332 57.6) (end 84.468 57.6) (width 0.4) (layer "F.Cu") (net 38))
 (segment (start 88.65 58.52) (end 88.65 57.918) (width 0.2) (layer "F.Cu") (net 38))
 (segment (start 88.65 57.981364) (end 88.65 57.918) (width 0.2) (layer "F.Cu") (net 38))
 (segment (start 88.95 58.281364) (end 88.65 57.981364) (width 0.2) (layer "F.Cu") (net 38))
 (segment (start 90.600394 62.853932) (end 90.478962 62.7325) (width 0.15) (layer "F.Cu") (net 38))
 (segment (start 88.332 57.6) (end 88.65 57.918) (width 0.2) (layer "F.Cu") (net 38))
 (segment (start 88.95 58.82) (end 88.95 58.281364) (width 0.2) (layer "F.Cu") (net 38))
 (segment (start 87.466018 61.384198) (end 87.61432 61.5325) (width 0.15) (layer "F.Cu") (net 38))
 (segment (start 84.468 57.6) (end 84.268 57.8) (width 0.4) (layer "F.Cu") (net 38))
 (segment (start 88.95 58.82) (end 88.65 58.52) (width 0.2) (layer "F.Cu") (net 38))
 (segment (start 84.15 57.918) (end 84.15 58.81) (width 0.3) (layer "F.Cu") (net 38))
 (segment (start 87.466018 61.384198) (end 86.601698 61.384198) (width 0.15) (layer "F.Cu") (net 38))
 (segment (start 83.85 58.81) (end 83.85 58.218) (width 0.2) (layer "F.Cu") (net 38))
 (segment (start 83.85 58.218) (end 84.268 57.8) (width 0.3) (layer "F.Cu") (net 38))
 (segment (start 88.65 57.918) (end 88.65 58.82) (width 0.2) (layer "F.Cu") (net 38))
 (segment (start 86.601698 61.384198) (end 86.6 61.3825) (width 0.15) (layer "F.Cu") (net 38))
 (segment (start 88.332 57.6) (end 88.2 57.6) (width 0.2) (layer "F.Cu") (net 38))
 (segment (start 87.61432 61.5325) (end 88.2 61.5325) (width 0.15) (layer "F.Cu") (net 38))
 (segment (start 90.478962 62.7325) (end 90.06 62.7325) (width 0.15) (layer "F.Cu") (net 38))
 (via (at 87.466018 61.384198) (size 0.6) (drill 0.3) (layers "F.Cu" "B.Cu") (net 38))
 (via (at 88.332 57.6) (size 0.6) (drill 0.3) (layers "F.Cu" "B.Cu") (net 38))
 (via (at 90.600394 62.853932) (size 0.6) (drill 0.3) (layers "F.Cu" "B.Cu") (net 38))
 (segment (start 87.466018 58.465982) (end 88.332 57.6) (width 0.4) (layer "B.Cu") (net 38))
 (segment (start 90.600394 62.853932) (end 90.600394 61.579638) (width 0.4) (layer "B.Cu") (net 38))
 (segment (start 87.466018 61.384198) (end 87.466018 58.465982) (width 0.4) (layer "B.Cu") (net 38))
 (segment (start 90.600394 61.579638) (end 90.404954 61.384198) (width 0.4) (layer "B.Cu") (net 38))
 (segment (start 90.404954 61.384198) (end 87.466018 61.384198) (width 0.4) (layer "B.Cu") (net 38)))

